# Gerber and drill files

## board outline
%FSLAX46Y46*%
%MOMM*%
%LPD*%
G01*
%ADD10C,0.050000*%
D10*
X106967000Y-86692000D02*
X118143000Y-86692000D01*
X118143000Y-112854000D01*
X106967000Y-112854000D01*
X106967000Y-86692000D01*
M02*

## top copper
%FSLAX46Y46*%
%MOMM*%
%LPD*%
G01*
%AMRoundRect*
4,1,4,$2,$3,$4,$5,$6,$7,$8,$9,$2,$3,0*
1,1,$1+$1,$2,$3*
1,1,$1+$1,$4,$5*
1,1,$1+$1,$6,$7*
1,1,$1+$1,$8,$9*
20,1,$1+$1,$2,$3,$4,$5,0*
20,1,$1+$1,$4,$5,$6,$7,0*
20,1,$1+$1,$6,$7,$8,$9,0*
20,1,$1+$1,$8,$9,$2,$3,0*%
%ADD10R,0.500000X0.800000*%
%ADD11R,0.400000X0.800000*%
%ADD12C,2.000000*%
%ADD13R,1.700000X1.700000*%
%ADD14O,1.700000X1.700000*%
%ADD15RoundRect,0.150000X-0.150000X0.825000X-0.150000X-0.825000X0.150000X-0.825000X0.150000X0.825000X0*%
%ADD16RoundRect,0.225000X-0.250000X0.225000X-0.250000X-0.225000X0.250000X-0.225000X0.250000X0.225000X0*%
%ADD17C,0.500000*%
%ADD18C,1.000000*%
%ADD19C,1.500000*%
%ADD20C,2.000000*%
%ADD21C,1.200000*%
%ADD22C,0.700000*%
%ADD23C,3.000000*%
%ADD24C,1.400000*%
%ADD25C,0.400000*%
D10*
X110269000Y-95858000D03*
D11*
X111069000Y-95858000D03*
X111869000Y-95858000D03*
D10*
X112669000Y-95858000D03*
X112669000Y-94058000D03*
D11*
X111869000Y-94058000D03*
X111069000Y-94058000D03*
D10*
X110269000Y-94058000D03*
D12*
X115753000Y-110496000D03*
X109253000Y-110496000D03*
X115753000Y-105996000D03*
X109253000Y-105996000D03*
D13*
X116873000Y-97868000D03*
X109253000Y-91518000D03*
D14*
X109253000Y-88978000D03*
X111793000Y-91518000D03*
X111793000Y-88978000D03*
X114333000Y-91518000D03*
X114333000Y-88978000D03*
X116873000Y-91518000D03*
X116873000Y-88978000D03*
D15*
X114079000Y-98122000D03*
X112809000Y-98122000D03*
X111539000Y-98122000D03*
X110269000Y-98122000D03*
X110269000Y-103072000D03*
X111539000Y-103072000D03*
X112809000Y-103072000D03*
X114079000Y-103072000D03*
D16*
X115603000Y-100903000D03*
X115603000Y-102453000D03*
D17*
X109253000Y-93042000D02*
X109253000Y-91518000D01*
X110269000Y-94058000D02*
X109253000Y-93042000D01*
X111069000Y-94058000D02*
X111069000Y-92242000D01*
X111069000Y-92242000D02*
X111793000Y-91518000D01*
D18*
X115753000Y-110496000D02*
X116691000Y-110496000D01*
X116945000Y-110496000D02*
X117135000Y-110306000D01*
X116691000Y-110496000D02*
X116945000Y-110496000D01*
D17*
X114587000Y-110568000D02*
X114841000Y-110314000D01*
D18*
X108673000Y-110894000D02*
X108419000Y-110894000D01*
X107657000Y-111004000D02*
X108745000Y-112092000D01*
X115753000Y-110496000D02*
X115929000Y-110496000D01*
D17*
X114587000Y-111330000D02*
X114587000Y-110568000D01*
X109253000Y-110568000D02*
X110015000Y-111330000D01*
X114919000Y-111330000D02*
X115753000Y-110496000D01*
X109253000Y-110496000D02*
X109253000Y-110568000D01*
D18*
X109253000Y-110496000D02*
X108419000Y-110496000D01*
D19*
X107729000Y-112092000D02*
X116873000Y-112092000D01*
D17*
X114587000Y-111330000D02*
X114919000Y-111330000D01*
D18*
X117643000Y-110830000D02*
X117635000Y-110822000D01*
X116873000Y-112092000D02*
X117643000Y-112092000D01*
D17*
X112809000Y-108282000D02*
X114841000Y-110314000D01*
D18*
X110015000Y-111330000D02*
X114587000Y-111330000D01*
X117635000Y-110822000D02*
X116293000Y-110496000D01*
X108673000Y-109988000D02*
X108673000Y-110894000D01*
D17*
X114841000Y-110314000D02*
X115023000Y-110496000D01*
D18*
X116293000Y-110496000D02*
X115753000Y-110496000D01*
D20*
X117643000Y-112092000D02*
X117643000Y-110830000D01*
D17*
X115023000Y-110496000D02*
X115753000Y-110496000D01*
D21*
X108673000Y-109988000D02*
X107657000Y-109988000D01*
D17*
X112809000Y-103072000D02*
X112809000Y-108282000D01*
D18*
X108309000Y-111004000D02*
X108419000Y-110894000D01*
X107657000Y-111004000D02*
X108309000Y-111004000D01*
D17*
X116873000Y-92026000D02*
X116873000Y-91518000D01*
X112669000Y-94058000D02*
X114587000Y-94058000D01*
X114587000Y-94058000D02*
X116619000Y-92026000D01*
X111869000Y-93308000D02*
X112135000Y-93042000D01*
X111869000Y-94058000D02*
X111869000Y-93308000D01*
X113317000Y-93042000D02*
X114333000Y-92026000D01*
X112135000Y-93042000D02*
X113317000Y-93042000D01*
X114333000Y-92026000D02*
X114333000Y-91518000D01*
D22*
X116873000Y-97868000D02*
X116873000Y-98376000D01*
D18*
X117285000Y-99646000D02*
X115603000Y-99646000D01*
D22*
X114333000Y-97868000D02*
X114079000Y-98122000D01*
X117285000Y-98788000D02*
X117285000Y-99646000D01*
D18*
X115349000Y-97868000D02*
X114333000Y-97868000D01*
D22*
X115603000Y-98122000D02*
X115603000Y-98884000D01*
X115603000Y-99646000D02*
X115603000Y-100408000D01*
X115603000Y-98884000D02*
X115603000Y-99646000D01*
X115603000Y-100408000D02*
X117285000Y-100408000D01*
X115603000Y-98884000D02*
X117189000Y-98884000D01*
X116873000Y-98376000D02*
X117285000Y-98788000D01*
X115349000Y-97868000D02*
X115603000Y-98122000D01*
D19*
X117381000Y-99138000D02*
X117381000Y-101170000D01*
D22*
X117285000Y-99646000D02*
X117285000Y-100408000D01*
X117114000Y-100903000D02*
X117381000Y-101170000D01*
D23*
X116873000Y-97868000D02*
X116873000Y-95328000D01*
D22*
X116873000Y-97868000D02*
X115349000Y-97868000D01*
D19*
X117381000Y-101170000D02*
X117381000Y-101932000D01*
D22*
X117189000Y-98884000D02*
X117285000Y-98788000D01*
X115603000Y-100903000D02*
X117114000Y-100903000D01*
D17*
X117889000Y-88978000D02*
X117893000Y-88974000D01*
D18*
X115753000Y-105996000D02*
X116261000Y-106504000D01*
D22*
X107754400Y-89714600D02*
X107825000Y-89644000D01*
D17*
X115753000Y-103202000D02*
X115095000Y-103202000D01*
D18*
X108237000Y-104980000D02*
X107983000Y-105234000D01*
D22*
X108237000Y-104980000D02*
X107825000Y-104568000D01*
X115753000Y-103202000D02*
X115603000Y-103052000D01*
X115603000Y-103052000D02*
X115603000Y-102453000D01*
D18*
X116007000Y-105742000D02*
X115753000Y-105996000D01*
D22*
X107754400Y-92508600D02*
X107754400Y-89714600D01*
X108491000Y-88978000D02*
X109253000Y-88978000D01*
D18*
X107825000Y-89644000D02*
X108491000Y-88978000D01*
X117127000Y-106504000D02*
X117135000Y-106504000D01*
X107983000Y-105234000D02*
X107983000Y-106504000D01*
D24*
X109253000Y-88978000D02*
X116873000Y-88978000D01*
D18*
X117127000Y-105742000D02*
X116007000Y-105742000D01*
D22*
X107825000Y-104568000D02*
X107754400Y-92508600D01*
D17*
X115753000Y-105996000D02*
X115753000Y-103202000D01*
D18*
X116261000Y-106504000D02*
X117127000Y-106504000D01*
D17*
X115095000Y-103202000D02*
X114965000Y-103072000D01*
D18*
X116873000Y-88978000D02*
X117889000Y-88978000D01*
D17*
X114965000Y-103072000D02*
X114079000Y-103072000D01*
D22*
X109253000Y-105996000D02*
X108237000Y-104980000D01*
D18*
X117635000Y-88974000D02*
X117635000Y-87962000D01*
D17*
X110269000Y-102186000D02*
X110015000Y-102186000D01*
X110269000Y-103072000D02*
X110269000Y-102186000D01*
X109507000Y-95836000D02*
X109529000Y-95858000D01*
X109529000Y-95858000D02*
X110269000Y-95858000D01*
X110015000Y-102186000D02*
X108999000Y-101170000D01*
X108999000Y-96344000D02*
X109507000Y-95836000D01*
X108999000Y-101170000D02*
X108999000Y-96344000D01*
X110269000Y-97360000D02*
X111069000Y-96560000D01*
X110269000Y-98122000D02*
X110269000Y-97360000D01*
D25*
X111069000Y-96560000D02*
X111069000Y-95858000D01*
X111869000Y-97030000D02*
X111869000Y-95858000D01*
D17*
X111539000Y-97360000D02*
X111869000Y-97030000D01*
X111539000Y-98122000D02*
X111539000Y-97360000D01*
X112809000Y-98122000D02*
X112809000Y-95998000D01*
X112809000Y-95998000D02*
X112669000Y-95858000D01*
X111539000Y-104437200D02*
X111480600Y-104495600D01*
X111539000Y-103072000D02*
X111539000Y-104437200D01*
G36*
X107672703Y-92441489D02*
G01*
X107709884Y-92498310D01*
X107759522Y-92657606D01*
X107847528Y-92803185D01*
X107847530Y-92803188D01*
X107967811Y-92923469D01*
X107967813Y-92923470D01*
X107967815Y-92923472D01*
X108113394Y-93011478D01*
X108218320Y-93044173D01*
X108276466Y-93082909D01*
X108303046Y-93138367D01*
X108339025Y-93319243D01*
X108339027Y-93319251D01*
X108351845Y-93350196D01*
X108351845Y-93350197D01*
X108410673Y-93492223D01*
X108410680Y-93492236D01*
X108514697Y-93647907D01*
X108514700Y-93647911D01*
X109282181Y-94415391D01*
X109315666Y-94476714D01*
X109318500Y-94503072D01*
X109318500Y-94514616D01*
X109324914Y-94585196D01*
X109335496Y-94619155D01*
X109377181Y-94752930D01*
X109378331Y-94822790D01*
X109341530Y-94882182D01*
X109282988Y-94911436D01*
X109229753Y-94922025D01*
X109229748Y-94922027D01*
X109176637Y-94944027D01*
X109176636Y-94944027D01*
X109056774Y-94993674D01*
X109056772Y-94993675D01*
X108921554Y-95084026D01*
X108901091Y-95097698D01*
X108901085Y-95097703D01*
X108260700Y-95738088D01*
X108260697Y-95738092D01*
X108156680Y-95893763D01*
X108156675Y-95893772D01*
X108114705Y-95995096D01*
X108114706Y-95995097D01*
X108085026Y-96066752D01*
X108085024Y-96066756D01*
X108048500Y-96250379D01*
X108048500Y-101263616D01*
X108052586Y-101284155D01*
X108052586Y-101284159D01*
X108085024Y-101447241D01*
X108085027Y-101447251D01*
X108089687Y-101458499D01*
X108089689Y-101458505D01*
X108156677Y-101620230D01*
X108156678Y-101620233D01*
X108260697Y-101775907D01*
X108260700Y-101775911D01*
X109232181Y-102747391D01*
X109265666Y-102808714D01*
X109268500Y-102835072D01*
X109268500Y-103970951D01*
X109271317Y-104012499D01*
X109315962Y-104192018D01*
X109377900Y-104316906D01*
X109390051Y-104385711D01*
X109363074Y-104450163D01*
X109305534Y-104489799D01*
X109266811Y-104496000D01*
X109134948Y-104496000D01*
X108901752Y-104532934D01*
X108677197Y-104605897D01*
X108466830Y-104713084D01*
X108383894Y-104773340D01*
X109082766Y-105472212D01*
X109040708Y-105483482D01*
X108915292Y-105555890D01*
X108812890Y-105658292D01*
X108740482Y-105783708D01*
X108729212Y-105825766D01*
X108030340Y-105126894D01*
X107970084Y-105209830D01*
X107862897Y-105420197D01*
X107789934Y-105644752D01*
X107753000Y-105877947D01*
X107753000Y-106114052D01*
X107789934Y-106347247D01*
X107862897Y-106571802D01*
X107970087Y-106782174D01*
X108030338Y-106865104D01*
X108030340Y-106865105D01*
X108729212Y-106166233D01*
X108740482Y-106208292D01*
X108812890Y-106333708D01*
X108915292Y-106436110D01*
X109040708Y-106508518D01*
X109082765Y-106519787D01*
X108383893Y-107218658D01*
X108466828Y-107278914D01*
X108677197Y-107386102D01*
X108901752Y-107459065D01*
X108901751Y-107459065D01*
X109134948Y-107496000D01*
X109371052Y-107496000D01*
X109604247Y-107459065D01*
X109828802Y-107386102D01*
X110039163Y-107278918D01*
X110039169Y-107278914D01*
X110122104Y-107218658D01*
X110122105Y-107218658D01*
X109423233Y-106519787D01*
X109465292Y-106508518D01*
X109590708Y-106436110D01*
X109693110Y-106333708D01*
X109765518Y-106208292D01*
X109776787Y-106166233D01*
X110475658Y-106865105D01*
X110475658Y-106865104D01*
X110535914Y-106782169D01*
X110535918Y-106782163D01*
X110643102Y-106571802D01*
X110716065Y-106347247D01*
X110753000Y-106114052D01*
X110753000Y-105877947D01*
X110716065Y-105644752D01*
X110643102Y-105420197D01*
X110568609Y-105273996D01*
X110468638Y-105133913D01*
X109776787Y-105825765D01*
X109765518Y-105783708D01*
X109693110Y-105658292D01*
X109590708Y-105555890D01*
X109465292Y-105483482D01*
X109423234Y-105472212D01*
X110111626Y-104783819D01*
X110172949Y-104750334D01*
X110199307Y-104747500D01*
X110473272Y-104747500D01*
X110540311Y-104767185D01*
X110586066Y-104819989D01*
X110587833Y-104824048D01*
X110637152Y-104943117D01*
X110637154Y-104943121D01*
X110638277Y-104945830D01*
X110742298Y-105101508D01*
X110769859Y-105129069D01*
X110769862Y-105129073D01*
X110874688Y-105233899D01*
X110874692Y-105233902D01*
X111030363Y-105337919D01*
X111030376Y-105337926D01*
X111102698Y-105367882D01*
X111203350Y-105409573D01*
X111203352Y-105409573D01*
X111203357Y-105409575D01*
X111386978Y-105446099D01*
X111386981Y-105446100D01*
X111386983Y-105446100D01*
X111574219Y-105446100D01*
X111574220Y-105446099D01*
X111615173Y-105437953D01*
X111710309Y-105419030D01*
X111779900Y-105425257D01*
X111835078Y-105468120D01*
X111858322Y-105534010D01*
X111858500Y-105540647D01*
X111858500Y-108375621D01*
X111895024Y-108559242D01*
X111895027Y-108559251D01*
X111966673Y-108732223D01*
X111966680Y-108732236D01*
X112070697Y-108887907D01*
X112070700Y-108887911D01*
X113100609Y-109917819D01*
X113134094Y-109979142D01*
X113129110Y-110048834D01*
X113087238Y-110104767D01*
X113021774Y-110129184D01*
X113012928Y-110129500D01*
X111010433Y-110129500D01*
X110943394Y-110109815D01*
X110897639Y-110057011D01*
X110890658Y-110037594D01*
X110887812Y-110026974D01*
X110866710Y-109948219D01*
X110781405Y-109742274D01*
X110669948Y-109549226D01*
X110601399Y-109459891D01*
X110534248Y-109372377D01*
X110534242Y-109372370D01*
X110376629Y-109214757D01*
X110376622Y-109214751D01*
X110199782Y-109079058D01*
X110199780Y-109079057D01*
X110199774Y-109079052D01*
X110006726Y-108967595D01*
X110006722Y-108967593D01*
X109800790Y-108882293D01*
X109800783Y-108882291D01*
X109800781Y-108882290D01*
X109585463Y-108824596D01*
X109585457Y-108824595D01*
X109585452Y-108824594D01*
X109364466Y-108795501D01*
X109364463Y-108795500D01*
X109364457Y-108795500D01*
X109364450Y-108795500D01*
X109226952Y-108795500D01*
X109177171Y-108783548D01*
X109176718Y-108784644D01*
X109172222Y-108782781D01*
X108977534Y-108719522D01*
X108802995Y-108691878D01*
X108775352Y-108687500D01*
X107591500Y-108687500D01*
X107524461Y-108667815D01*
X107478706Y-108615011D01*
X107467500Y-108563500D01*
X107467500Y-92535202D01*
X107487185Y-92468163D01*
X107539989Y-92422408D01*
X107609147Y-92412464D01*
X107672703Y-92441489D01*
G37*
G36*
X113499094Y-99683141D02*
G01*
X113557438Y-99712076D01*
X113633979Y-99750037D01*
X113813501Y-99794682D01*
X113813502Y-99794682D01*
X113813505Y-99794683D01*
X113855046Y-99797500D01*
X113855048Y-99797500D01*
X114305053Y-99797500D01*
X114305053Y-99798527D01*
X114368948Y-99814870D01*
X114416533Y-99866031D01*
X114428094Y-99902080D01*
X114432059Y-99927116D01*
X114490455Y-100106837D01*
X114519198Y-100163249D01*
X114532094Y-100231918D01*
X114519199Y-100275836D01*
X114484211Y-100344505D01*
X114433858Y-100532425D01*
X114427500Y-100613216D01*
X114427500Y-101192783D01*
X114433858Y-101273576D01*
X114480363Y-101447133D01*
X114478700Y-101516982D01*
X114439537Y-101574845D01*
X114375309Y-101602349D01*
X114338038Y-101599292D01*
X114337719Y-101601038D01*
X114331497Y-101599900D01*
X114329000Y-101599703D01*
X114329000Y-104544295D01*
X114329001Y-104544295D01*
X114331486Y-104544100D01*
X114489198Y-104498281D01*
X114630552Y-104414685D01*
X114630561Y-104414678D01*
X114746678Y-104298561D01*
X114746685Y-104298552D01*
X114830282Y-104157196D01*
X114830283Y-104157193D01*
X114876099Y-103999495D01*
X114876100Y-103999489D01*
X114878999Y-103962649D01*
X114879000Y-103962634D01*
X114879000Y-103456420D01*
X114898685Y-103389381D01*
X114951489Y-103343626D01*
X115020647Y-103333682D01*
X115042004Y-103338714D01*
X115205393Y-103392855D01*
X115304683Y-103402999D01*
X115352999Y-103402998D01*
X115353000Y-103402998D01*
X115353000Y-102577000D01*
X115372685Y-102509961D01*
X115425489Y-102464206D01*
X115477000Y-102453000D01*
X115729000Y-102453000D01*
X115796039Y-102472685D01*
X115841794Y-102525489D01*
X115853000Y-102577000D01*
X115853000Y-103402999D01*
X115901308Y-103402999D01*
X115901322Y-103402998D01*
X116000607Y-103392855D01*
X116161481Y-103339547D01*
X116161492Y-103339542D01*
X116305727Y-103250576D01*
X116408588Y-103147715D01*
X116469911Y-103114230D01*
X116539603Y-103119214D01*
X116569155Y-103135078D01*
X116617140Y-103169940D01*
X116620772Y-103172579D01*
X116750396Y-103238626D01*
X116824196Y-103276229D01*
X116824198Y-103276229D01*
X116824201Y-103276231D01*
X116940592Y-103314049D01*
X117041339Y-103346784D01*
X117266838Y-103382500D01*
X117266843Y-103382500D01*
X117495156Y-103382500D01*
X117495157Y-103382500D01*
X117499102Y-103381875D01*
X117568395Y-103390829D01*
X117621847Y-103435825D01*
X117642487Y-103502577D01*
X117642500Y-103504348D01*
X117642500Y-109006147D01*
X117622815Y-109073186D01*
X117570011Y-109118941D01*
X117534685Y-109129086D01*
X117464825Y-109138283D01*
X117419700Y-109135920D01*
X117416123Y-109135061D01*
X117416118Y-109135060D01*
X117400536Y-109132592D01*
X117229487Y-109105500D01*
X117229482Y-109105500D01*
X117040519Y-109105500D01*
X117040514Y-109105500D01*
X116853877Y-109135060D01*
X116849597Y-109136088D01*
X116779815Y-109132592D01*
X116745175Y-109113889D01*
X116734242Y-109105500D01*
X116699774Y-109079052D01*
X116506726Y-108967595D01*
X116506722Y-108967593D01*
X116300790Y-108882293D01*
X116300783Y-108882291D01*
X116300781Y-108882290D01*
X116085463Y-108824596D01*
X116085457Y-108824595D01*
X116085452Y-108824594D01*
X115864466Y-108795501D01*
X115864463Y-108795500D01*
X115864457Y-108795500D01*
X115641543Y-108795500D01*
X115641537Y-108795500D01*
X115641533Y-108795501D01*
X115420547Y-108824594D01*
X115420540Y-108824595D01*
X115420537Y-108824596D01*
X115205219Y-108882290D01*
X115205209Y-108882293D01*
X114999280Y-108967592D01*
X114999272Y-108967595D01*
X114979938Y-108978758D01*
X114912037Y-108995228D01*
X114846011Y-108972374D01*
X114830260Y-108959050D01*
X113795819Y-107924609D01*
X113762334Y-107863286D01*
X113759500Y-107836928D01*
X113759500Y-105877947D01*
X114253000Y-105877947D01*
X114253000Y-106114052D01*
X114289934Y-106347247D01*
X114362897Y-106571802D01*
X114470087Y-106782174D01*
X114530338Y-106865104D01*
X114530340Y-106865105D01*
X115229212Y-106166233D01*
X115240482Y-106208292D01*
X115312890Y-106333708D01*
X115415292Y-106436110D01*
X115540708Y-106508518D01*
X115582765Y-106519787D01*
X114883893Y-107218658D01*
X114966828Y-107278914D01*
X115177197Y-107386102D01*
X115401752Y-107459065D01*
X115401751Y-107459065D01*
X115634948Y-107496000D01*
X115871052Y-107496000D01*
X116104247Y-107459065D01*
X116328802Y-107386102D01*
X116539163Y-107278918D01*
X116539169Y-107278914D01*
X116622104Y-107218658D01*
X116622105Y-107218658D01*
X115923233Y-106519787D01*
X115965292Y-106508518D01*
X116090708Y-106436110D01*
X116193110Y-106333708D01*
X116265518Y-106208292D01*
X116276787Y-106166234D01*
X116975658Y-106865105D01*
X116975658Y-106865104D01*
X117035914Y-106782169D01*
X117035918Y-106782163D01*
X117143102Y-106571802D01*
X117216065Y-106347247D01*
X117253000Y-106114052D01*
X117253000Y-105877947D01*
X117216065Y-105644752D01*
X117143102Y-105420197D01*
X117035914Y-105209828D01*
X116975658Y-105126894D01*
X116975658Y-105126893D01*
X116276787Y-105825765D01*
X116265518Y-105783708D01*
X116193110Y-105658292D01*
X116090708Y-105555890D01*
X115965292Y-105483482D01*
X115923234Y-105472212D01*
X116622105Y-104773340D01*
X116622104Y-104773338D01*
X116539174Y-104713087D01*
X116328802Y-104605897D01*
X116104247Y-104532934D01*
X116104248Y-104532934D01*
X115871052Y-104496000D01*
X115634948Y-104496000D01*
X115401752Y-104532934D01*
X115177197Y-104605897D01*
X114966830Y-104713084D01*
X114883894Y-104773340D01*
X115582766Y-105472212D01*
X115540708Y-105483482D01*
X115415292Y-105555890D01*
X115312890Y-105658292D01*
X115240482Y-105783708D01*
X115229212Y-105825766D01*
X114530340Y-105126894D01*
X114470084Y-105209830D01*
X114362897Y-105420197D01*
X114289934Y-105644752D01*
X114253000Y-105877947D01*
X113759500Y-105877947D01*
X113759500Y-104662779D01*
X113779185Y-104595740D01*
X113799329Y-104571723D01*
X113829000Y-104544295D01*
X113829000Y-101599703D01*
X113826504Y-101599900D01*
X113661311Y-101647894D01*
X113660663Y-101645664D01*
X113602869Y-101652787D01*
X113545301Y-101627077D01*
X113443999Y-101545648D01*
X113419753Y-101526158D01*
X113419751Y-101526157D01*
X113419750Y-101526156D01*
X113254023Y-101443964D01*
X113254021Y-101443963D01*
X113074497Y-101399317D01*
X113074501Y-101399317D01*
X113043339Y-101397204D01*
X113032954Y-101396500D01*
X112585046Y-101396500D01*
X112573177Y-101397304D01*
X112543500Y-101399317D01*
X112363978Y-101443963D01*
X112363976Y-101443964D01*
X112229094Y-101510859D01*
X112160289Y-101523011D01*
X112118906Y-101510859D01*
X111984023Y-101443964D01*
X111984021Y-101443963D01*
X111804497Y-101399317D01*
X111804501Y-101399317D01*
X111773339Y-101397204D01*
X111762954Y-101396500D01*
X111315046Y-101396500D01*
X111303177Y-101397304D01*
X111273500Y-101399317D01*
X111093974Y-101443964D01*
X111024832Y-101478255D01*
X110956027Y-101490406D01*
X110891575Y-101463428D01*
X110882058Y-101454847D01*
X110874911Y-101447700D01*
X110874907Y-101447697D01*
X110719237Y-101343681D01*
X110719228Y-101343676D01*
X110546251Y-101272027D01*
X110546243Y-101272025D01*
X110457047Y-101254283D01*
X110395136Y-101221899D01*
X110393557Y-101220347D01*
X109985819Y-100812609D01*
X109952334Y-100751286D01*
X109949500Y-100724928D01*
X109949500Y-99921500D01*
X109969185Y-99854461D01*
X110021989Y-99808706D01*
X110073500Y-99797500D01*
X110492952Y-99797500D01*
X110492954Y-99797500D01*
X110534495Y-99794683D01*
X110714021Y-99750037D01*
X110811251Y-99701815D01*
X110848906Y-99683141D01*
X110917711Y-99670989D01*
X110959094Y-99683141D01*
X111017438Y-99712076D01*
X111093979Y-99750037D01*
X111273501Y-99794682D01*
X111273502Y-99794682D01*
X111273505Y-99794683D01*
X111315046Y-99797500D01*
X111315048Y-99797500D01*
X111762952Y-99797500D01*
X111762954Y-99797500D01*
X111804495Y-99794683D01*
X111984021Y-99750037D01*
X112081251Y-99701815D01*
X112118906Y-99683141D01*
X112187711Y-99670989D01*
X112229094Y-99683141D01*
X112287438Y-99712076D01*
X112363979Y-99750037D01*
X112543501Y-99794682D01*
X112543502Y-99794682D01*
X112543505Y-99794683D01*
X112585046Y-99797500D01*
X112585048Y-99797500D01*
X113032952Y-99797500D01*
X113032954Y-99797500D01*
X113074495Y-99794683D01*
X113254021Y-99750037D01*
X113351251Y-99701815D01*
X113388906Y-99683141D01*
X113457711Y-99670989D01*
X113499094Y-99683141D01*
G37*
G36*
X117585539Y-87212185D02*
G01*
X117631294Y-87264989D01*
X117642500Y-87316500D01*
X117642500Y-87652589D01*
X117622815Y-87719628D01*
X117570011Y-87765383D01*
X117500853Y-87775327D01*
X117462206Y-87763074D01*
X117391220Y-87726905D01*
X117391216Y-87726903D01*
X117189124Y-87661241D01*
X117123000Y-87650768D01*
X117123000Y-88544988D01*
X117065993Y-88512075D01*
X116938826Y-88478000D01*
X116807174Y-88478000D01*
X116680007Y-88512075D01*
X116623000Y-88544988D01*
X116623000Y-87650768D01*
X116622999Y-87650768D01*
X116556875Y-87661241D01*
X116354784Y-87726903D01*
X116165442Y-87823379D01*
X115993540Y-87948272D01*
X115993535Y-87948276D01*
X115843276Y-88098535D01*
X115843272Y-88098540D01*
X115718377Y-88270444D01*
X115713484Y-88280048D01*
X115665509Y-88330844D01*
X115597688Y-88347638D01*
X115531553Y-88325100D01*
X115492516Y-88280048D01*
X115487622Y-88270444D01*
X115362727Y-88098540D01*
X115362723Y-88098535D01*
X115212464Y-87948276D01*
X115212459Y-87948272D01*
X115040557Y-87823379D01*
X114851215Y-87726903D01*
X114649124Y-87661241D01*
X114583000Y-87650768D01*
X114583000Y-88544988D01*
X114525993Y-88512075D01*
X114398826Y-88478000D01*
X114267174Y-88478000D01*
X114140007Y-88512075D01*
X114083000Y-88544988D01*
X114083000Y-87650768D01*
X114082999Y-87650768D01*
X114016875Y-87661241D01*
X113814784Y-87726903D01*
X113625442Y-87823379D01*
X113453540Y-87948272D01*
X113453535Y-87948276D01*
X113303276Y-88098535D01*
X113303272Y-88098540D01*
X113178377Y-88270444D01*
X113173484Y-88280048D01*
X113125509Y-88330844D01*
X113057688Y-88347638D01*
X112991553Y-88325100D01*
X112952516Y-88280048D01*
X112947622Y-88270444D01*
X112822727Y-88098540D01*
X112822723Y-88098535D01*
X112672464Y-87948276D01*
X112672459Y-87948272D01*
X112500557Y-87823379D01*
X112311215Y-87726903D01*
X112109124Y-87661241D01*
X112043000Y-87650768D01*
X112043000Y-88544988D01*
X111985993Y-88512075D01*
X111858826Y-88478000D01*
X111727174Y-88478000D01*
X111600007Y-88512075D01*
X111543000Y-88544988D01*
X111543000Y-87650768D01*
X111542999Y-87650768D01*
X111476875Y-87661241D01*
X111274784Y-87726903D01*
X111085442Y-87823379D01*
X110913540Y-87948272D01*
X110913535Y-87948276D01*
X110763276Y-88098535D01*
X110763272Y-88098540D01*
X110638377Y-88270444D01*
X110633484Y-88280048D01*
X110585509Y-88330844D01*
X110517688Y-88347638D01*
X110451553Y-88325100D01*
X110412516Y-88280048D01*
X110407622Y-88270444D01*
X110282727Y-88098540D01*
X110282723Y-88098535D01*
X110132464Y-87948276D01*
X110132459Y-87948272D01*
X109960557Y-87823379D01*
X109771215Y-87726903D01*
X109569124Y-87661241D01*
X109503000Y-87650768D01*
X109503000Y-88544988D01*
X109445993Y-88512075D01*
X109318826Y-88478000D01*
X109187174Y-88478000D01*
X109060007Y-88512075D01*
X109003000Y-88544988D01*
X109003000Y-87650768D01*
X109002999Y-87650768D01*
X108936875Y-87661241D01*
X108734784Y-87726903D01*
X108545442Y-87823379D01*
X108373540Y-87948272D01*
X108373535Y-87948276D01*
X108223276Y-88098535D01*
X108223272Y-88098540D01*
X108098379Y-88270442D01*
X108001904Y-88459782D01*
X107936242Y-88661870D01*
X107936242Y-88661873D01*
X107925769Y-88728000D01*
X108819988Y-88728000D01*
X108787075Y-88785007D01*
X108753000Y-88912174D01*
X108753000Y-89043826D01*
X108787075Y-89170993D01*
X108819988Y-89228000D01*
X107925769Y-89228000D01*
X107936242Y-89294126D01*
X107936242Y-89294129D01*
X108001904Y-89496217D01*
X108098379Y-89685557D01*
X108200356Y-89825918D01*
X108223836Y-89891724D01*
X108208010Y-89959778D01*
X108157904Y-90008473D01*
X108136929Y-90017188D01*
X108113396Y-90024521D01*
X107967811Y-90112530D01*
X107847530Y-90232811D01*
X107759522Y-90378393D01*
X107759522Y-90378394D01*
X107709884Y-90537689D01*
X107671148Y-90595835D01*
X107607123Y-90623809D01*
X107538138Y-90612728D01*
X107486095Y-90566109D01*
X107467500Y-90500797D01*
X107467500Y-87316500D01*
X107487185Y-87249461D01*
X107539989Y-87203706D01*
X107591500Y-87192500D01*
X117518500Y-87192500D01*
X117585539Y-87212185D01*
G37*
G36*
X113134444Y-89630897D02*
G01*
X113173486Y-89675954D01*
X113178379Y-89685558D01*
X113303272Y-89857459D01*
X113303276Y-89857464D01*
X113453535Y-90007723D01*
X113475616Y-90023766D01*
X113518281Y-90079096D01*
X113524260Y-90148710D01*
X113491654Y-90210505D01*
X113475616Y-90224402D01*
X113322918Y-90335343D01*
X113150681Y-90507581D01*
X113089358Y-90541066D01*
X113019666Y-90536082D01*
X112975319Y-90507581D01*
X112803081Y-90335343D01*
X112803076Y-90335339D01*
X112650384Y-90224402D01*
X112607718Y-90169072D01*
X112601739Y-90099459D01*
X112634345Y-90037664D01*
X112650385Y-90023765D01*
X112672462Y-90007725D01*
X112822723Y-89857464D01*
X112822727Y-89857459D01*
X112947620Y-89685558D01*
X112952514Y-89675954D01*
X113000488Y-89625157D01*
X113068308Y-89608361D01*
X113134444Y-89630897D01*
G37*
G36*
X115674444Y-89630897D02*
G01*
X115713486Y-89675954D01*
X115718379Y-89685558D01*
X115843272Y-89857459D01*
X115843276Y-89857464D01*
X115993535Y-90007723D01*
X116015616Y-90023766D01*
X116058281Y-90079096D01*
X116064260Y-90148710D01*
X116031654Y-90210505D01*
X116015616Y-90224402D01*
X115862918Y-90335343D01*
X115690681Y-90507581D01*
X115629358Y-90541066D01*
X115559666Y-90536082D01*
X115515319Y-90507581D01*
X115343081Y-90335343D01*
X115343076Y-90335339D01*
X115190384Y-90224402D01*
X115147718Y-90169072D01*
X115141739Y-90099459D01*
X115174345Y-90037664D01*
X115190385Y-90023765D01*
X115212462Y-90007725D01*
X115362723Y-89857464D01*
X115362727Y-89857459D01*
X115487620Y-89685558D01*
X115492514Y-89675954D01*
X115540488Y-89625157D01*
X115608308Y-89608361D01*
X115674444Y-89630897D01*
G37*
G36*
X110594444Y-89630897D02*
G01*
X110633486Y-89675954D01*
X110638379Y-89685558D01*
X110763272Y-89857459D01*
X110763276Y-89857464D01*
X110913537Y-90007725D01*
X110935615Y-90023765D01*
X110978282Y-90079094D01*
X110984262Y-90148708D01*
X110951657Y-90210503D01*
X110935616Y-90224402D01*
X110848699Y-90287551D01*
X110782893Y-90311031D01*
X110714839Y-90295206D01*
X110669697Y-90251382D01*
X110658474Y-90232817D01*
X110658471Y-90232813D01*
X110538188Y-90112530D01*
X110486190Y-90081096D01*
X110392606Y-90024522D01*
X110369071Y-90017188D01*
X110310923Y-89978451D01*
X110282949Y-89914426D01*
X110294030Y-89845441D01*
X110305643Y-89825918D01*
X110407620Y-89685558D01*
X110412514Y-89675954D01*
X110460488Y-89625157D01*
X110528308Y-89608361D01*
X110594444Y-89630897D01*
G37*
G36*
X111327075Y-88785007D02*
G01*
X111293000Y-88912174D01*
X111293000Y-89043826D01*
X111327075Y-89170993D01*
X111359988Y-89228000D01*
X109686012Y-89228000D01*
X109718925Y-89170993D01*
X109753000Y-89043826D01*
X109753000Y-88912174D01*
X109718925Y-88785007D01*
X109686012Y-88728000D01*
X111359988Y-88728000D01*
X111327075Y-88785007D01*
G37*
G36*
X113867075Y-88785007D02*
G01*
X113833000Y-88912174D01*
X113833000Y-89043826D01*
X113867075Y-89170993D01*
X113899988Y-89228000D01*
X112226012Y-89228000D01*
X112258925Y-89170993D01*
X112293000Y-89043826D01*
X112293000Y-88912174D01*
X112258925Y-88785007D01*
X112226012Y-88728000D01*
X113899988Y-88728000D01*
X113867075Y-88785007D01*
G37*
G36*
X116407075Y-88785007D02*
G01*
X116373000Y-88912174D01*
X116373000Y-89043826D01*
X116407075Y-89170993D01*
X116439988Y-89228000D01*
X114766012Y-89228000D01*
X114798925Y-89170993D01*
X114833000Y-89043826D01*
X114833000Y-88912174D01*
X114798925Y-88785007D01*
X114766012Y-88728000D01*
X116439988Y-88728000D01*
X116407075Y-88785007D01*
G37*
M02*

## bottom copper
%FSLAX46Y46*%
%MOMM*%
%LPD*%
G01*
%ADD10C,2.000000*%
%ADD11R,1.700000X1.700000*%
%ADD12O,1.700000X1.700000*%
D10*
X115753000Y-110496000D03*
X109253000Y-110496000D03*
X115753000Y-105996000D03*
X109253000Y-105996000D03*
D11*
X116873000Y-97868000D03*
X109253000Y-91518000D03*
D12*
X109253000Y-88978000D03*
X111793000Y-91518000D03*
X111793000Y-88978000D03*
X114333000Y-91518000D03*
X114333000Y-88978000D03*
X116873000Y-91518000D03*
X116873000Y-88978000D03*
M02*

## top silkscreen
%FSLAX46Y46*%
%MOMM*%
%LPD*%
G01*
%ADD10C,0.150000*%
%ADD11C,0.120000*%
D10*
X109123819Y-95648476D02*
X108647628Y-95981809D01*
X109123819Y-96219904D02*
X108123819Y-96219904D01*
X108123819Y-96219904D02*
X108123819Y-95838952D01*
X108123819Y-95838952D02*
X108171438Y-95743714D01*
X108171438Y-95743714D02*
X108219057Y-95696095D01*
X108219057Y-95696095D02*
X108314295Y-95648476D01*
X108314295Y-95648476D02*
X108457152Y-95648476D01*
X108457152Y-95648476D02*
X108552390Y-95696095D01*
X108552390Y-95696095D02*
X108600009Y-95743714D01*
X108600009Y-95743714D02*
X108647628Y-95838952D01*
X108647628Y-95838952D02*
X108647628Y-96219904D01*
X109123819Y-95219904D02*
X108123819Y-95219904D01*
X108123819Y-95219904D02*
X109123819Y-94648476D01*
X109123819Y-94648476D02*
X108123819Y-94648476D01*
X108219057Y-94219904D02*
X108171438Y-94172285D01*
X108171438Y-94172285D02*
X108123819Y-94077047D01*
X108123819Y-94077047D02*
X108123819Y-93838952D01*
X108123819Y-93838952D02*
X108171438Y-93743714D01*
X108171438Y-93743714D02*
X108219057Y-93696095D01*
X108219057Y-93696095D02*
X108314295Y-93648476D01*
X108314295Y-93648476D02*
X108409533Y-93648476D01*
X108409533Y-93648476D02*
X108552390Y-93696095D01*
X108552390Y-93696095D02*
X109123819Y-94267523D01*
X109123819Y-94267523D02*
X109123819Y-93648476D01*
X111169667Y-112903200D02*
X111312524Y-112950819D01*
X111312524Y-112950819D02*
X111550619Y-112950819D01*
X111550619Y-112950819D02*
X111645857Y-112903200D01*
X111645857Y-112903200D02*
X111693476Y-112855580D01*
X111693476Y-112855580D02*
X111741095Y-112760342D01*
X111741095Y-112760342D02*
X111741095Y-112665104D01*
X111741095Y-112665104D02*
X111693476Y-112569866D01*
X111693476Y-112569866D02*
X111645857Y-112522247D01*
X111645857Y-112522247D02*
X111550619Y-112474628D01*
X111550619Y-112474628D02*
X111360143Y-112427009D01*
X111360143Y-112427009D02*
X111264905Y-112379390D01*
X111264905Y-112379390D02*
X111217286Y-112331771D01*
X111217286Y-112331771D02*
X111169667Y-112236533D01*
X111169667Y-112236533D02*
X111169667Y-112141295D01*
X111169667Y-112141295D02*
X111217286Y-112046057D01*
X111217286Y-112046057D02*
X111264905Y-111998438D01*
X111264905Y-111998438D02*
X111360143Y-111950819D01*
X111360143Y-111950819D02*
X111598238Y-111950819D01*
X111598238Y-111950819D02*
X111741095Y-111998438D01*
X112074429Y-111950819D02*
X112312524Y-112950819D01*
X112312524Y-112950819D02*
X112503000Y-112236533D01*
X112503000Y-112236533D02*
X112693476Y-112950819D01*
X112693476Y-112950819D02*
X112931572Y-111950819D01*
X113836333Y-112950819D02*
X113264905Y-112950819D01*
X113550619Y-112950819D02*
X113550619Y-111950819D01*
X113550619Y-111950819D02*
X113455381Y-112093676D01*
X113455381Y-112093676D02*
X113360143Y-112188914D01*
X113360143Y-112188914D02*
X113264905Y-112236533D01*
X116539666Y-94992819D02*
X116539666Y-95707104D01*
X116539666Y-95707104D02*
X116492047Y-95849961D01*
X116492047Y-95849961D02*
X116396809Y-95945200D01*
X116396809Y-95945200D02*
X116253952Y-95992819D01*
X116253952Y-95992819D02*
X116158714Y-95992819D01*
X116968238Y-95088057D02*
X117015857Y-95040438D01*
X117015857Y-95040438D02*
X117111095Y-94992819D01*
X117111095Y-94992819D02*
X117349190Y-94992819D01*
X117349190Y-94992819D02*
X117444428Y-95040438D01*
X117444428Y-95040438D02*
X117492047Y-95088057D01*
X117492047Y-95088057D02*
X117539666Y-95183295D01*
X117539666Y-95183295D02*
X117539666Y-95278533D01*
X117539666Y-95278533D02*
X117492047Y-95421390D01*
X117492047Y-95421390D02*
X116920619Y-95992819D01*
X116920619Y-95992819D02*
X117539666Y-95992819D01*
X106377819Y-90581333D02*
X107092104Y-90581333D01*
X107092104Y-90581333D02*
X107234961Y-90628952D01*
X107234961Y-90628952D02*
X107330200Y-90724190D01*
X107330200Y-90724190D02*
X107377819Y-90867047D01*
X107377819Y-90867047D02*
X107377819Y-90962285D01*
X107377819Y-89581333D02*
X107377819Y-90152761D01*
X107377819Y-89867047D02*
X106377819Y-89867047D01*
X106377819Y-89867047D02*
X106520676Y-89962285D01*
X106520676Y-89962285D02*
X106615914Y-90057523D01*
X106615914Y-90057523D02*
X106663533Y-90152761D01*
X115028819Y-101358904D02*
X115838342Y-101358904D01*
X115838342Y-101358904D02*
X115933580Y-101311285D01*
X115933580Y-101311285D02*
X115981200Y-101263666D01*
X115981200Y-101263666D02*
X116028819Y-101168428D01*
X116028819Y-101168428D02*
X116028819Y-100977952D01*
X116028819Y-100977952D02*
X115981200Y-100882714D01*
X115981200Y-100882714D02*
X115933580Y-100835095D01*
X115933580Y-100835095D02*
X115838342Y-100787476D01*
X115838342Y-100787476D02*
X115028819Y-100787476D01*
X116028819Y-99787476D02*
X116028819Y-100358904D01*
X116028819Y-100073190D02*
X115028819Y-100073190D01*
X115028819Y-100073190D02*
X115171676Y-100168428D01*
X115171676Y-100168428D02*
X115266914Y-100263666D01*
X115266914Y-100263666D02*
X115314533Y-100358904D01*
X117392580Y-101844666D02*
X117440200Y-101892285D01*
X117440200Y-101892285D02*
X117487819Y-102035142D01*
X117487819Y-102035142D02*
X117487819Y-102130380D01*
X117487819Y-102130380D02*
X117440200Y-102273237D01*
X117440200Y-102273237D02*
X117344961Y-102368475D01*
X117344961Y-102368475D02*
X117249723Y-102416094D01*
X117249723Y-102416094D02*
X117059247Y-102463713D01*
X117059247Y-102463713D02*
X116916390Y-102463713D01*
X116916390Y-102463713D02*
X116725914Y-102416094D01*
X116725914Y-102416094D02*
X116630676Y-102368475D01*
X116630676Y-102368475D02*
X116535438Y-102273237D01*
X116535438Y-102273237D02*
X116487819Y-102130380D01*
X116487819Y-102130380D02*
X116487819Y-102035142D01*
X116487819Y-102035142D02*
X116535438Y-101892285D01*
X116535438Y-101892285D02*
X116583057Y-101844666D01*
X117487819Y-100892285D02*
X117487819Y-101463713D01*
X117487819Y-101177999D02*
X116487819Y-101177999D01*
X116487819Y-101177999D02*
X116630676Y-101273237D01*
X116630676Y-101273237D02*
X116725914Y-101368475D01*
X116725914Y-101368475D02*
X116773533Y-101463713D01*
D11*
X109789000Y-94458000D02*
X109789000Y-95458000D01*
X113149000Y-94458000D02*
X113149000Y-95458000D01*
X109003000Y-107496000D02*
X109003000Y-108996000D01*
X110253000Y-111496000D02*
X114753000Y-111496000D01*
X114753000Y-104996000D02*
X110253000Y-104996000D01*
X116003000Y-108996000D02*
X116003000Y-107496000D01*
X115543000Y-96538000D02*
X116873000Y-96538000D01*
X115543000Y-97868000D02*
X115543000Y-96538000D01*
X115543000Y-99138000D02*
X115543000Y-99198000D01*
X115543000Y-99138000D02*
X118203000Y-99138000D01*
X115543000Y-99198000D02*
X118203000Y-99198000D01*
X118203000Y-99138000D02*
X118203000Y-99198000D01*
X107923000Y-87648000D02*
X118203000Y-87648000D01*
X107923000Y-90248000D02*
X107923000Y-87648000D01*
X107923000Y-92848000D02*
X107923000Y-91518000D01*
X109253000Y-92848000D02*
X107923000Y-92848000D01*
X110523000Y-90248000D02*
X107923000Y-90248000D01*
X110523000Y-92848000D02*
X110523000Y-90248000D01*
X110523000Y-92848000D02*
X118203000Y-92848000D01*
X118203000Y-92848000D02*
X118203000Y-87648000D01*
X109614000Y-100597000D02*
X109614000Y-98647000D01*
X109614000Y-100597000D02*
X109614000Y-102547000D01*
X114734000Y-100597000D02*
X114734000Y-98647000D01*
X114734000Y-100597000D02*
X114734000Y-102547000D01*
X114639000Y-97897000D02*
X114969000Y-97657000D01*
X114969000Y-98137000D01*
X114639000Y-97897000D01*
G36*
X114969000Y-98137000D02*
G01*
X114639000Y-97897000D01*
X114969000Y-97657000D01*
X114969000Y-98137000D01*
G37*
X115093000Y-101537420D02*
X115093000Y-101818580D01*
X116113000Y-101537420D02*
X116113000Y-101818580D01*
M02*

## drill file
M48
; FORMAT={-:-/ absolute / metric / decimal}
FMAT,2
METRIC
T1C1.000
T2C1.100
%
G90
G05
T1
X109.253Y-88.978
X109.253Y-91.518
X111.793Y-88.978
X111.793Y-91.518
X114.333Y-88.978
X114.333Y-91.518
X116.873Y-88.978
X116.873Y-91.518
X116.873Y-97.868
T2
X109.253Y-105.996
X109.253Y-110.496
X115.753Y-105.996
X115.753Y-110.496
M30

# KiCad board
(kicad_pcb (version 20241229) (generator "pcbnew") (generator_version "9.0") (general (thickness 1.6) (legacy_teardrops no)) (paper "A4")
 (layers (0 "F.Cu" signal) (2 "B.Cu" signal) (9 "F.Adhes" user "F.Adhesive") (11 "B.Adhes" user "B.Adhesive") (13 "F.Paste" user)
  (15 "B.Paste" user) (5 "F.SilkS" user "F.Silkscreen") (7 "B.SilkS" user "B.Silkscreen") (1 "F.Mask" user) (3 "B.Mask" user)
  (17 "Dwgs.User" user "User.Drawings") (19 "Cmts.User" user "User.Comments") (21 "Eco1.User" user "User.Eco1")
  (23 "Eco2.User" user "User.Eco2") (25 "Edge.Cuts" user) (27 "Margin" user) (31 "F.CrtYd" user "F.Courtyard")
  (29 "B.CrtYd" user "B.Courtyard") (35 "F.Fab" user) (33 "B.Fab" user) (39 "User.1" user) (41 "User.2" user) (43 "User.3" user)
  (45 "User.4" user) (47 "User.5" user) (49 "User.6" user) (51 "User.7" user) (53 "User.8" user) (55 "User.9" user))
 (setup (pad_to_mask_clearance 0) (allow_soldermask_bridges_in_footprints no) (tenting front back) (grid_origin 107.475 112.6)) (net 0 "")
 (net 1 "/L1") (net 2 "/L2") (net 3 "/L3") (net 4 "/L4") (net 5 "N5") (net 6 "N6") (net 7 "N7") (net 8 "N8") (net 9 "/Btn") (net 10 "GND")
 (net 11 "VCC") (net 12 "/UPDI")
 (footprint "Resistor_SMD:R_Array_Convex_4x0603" (layer "F.Cu") (at 111.469 94.958 90)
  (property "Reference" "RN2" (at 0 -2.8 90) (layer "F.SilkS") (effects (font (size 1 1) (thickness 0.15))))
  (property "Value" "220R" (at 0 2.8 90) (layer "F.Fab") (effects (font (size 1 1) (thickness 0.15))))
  (fp_line (start 0.5 -1.68) (end -0.5 -1.68) (stroke (width 0.12) (type solid)) (layer "F.SilkS"))
  (fp_line (start 0.5 1.68) (end -0.5 1.68) (stroke (width 0.12) (type solid)) (layer "F.SilkS"))
  (pad "1" smd rect (at -0.9 -1.2 90) (size 0.8 0.5) (layers "F.Cu" "F.Mask" "F.Paste") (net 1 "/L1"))
  (pad "2" smd rect (at -0.9 -0.4 90) (size 0.8 0.4) (layers "F.Cu" "F.Mask" "F.Paste") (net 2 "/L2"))
  (pad "3" smd rect (at -0.9 0.4 90) (size 0.8 0.4) (layers "F.Cu" "F.Mask" "F.Paste") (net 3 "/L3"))
  (pad "4" smd rect (at -0.9 1.2 90) (size 0.8 0.5) (layers "F.Cu" "F.Mask" "F.Paste") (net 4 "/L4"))
  (pad "5" smd rect (at 0.9 1.2 90) (size 0.8 0.5) (layers "F.Cu" "F.Mask" "F.Paste") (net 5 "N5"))
  (pad "6" smd rect (at 0.9 0.4 90) (size 0.8 0.4) (layers "F.Cu" "F.Mask" "F.Paste") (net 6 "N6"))
  (pad "7" smd rect (at 0.9 -0.4 90) (size 0.8 0.4) (layers "F.Cu" "F.Mask" "F.Paste") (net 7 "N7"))
  (pad "8" smd rect (at 0.9 -1.2 90) (size 0.8 0.5) (layers "F.Cu" "F.Mask" "F.Paste") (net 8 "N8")))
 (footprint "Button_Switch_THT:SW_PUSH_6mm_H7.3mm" (layer "F.Cu") (at 115.753 110.496 180)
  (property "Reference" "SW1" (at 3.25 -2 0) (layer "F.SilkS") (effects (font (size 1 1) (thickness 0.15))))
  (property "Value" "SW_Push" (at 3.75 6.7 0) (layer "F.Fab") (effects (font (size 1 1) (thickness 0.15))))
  (fp_line (start 6.75 3) (end 6.75 1.5) (stroke (width 0.12) (type solid)) (layer "F.SilkS"))
  (fp_line (start 5.5 -1) (end 1 -1) (stroke (width 0.12) (type solid)) (layer "F.SilkS"))
  (fp_line (start 1 5.5) (end 5.5 5.5) (stroke (width 0.12) (type solid)) (layer "F.SilkS"))
  (fp_line (start -0.25 1.5) (end -0.25 3) (stroke (width 0.12) (type solid)) (layer "F.SilkS"))
  (pad "1" thru_hole circle (at 0 0 270) (size 2 2) (drill 1.1) (layers "*.Cu" "*.Mask") (remove_unused_layers no) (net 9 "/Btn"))
  (pad "1" thru_hole circle (at 6.5 0 270) (size 2 2) (drill 1.1) (layers "*.Cu" "*.Mask") (remove_unused_layers no) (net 9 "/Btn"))
  (pad "2" thru_hole circle (at 0 4.5 270) (size 2 2) (drill 1.1) (layers "*.Cu" "*.Mask") (remove_unused_layers no) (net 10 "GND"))
  (pad "2" thru_hole circle (at 6.5 4.5 270) (size 2 2) (drill 1.1) (layers "*.Cu" "*.Mask") (remove_unused_layers no) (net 10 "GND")))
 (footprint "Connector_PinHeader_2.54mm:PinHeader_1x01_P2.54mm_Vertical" (layer "F.Cu") (at 116.873 97.868)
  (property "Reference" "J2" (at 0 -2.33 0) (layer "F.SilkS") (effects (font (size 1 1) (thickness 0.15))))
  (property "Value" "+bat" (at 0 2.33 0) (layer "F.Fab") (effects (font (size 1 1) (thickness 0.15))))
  (fp_line (start -1.33 -1.33) (end 0 -1.33) (stroke (width 0.12) (type solid)) (layer "F.SilkS"))
  (fp_line (start -1.33 0) (end -1.33 -1.33) (stroke (width 0.12) (type solid)) (layer "F.SilkS"))
  (fp_line (start -1.33 1.27) (end -1.33 1.33) (stroke (width 0.12) (type solid)) (layer "F.SilkS"))
  (fp_line (start -1.33 1.27) (end 1.33 1.27) (stroke (width 0.12) (type solid)) (layer "F.SilkS"))
  (fp_line (start -1.33 1.33) (end 1.33 1.33) (stroke (width 0.12) (type solid)) (layer "F.SilkS"))
  (fp_line (start 1.33 1.27) (end 1.33 1.33) (stroke (width 0.12) (type solid)) (layer "F.SilkS"))
  (pad "1" thru_hole rect (at 0 0) (size 1.7 1.7) (drill 1) (layers "*.Cu" "*.Mask") (remove_unused_layers no) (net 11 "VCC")))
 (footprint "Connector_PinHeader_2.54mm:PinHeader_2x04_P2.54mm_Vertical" (layer "F.Cu") (at 109.253 91.518 90)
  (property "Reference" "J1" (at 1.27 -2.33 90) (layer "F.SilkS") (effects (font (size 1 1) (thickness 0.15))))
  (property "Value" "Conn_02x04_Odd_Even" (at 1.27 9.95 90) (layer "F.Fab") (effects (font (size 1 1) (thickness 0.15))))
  (fp_line (start 3.87 -1.33) (end 3.87 8.95) (stroke (width 0.12) (type solid)) (layer "F.SilkS"))
  (fp_line (start 1.27 -1.33) (end 3.87 -1.33) (stroke (width 0.12) (type solid)) (layer "F.SilkS"))
  (fp_line (start -1.33 -1.33) (end 0 -1.33) (stroke (width 0.12) (type solid)) (layer "F.SilkS"))
  (fp_line (start -1.33 0) (end -1.33 -1.33) (stroke (width 0.12) (type solid)) (layer "F.SilkS"))
  (fp_line (start 1.27 1.27) (end 1.27 -1.33) (stroke (width 0.12) (type solid)) (layer "F.SilkS"))
  (fp_line (start -1.33 1.27) (end 1.27 1.27) (stroke (width 0.12) (type solid)) (layer "F.SilkS"))
  (fp_line (start -1.33 1.27) (end -1.33 8.95) (stroke (width 0.12) (type solid)) (layer "F.SilkS"))
  (fp_line (start -1.33 8.95) (end 3.87 8.95) (stroke (width 0.12) (type solid)) (layer "F.SilkS"))
  (pad "1" thru_hole rect (at 0 0 90) (size 1.7 1.7) (drill 1) (layers "*.Cu" "*.Mask") (remove_unused_layers no) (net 8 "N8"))
  (pad "2" thru_hole oval (at 2.54 0 90) (size 1.7 1.7) (drill 1) (layers "*.Cu" "*.Mask") (remove_unused_layers no) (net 10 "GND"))
  (pad "3" thru_hole oval (at 0 2.54 90) (size 1.7 1.7) (drill 1) (layers "*.Cu" "*.Mask") (remove_unused_layers no) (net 7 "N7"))
  (pad "4" thru_hole oval (at 2.54 2.54 90) (size 1.7 1.7) (drill 1) (layers "*.Cu" "*.Mask") (remove_unused_layers no) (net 10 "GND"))
  (pad "5" thru_hole oval (at 0 5.08 90) (size 1.7 1.7) (drill 1) (layers "*.Cu" "*.Mask") (remove_unused_layers no) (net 6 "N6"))
  (pad "6" thru_hole oval (at 2.54 5.08 90) (size 1.7 1.7) (drill 1) (layers "*.Cu" "*.Mask") (remove_unused_layers no) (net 10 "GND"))
  (pad "7" thru_hole oval (at 0 7.62 90) (size 1.7 1.7) (drill 1) (layers "*.Cu" "*.Mask") (remove_unused_layers no) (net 5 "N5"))
  (pad "8" thru_hole oval (at 2.54 7.62 90) (size 1.7 1.7) (drill 1) (layers "*.Cu" "*.Mask") (remove_unused_layers no) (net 10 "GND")))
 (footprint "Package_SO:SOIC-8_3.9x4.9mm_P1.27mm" (layer "F.Cu") (at 112.174 100.597 -90)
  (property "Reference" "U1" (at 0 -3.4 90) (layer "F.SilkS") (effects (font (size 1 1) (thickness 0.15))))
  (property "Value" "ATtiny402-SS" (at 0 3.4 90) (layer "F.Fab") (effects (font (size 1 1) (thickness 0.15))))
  (fp_line (start 0 2.56) (end -1.95 2.56) (stroke (width 0.12) (type solid)) (layer "F.SilkS"))
  (fp_line (start 0 2.56) (end 1.95 2.56) (stroke (width 0.12) (type solid)) (layer "F.SilkS"))
  (fp_line (start 0 -2.56) (end -1.95 -2.56) (stroke (width 0.12) (type solid)) (layer "F.SilkS"))
  (fp_line (start 0 -2.56) (end 1.95 -2.56) (stroke (width 0.12) (type solid)) (layer "F.SilkS"))
  (fp_poly
   (pts (xy -2.7 -2.465) (xy -2.94 -2.795) (xy -2.46 -2.795) (xy -2.7 -2.465)) (stroke (width 0.12) (type solid)) (fill yes)
   (layer "F.SilkS"))
  (pad "1" smd roundrect (at -2.475 -1.905 270) (size 1.95 0.6) (layers "F.Cu" "F.Mask" "F.Paste") (roundrect_rratio 0.25) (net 11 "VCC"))
  (pad "2" smd roundrect (at -2.475 -0.635 270) (size 1.95 0.6) (layers "F.Cu" "F.Mask" "F.Paste") (roundrect_rratio 0.25) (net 4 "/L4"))
  (pad "3" smd roundrect (at -2.475 0.635 270) (size 1.95 0.6) (layers "F.Cu" "F.Mask" "F.Paste") (roundrect_rratio 0.25) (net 3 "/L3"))
  (pad "4" smd roundrect (at -2.475 1.905 270) (size 1.95 0.6) (layers "F.Cu" "F.Mask" "F.Paste") (roundrect_rratio 0.25) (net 2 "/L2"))
  (pad "5" smd roundrect (at 2.475 1.905 270) (size 1.95 0.6) (layers "F.Cu" "F.Mask" "F.Paste") (roundrect_rratio 0.25) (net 1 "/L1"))
  (pad "6" smd roundrect (at 2.475 0.635 270) (size 1.95 0.6) (layers "F.Cu" "F.Mask" "F.Paste") (roundrect_rratio 0.25) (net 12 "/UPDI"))
  (pad "7" smd roundrect (at 2.475 -0.635 270) (size 1.95 0.6) (layers "F.Cu" "F.Mask" "F.Paste") (roundrect_rratio 0.25) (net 9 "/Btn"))
  (pad "8" smd roundrect (at 2.475 -1.905 270) (size 1.95 0.6) (layers "F.Cu" "F.Mask" "F.Paste") (roundrect_rratio 0.25) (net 10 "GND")))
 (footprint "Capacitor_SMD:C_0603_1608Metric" (layer "F.Cu") (at 115.603 101.678 -90)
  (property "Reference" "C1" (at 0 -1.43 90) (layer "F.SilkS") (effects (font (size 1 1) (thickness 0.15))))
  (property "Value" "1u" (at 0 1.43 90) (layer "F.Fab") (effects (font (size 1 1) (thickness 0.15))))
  (fp_line (start -0.14058 0.51) (end 0.14058 0.51) (stroke (width 0.12) (type solid)) (layer "F.SilkS"))
  (fp_line (start -0.14058 -0.51) (end 0.14058 -0.51) (stroke (width 0.12) (type solid)) (layer "F.SilkS"))
  (pad "1" smd roundrect (at -0.775 0 270) (size 0.9 0.95) (layers "F.Cu" "F.Mask" "F.Paste") (roundrect_rratio 0.25) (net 11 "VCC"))
  (pad "2" smd roundrect (at 0.775 0 270) (size 0.9 0.95) (layers "F.Cu" "F.Mask" "F.Paste") (roundrect_rratio 0.25) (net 10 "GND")))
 (gr_rect (start 106.967 86.692) (end 118.143 112.854) (stroke (width 0.05) (type default)) (fill no) (layer "Edge.Cuts"))
 (segment (start 109.253 93.042) (end 109.253 91.518) (width 0.5) (layer "F.Cu") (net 8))
 (segment (start 110.269 94.058) (end 109.253 93.042) (width 0.5) (layer "F.Cu") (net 8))
 (segment (start 111.069 94.058) (end 111.069 92.242) (width 0.5) (layer "F.Cu") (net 7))
 (segment (start 111.069 92.242) (end 111.793 91.518) (width 0.5) (layer "F.Cu") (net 7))
 (segment (start 115.753 110.496) (end 116.691 110.496) (width 1) (layer "F.Cu") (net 9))
 (segment (start 116.945 110.496) (end 117.135 110.306) (width 1) (layer "F.Cu") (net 9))
 (segment (start 116.691 110.496) (end 116.945 110.496) (width 1) (layer "F.Cu") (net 9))
 (segment (start 114.587 110.568) (end 114.841 110.314) (width 0.5) (layer "F.Cu") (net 9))
 (segment (start 108.673 110.894) (end 108.419 110.894) (width 1) (layer "F.Cu") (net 9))
 (segment (start 107.657 111.004) (end 108.745 112.092) (width 1) (layer "F.Cu") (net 9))
 (segment (start 115.753 110.496) (end 115.929 110.496) (width 1) (layer "F.Cu") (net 9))
 (segment (start 114.587 111.33) (end 114.587 110.568) (width 0.5) (layer "F.Cu") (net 9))
 (segment (start 109.253 110.568) (end 110.015 111.33) (width 0.5) (layer "F.Cu") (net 9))
 (segment (start 114.919 111.33) (end 115.753 110.496) (width 0.5) (layer "F.Cu") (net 9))
 (segment (start 109.253 110.496) (end 109.253 110.568) (width 0.5) (layer "F.Cu") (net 9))
 (segment (start 109.253 110.496) (end 108.419 110.496) (width 1) (layer "F.Cu") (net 9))
 (segment (start 107.729 112.092) (end 116.873 112.092) (width 1.5) (layer "F.Cu") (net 9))
 (segment (start 114.587 111.33) (end 114.919 111.33) (width 0.5) (layer "F.Cu") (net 9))
 (segment (start 117.643 110.83) (end 117.635 110.822) (width 1) (layer "F.Cu") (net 9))
 (segment (start 116.873 112.092) (end 117.643 112.092) (width 1) (layer "F.Cu") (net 9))
 (segment (start 112.809 108.282) (end 114.841 110.314) (width 0.5) (layer "F.Cu") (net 9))
 (segment (start 110.015 111.33) (end 114.587 111.33) (width 1) (layer "F.Cu") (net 9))
 (segment (start 117.635 110.822) (end 116.293 110.496) (width 1) (layer "F.Cu") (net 9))
 (segment (start 108.673 109.988) (end 108.673 110.894) (width 1) (layer "F.Cu") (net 9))
 (segment (start 114.841 110.314) (end 115.023 110.496) (width 0.5) (layer "F.Cu") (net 9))
 (segment (start 116.293 110.496) (end 115.753 110.496) (width 1) (layer "F.Cu") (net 9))
 (segment (start 117.643 112.092) (end 117.643 110.83) (width 2) (layer "F.Cu") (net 9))
 (segment (start 115.023 110.496) (end 115.753 110.496) (width 0.5) (layer "F.Cu") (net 9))
 (segment (start 108.673 109.988) (end 107.657 109.988) (width 1.2) (layer "F.Cu") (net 9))
 (segment (start 112.809 103.072) (end 112.809 108.282) (width 0.5) (layer "F.Cu") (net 9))
 (segment (start 108.309 111.004) (end 108.419 110.894) (width 1) (layer "F.Cu") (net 9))
 (segment (start 107.657 111.004) (end 108.309 111.004) (width 1) (layer "F.Cu") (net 9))
 (segment (start 116.873 92.026) (end 116.873 91.518) (width 0.5) (layer "F.Cu") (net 5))
 (segment (start 112.669 94.058) (end 114.587 94.058) (width 0.5) (layer "F.Cu") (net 5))
 (segment (start 114.587 94.058) (end 116.619 92.026) (width 0.5) (layer "F.Cu") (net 5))
 (segment (start 111.869 93.308) (end 112.135 93.042) (width 0.5) (layer "F.Cu") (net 6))
 (segment (start 111.869 94.058) (end 111.869 93.308) (width 0.5) (layer "F.Cu") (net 6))
 (segment (start 113.317 93.042) (end 114.333 92.026) (width 0.5) (layer "F.Cu") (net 6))
 (segment (start 112.135 93.042) (end 113.317 93.042) (width 0.5) (layer "F.Cu") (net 6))
 (segment (start 114.333 92.026) (end 114.333 91.518) (width 0.5) (layer "F.Cu") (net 6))
 (segment (start 116.873 97.868) (end 116.873 98.376) (width 0.7) (layer "F.Cu") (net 11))
 (segment (start 117.285 99.646) (end 115.603 99.646) (width 1) (layer "F.Cu") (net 11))
 (segment (start 114.333 97.868) (end 114.079 98.122) (width 0.7) (layer "F.Cu") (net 11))
 (segment (start 117.285 98.788) (end 117.285 99.646) (width 0.7) (layer "F.Cu") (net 11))
 (segment (start 115.349 97.868) (end 114.333 97.868) (width 1) (layer "F.Cu") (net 11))
 (segment (start 115.603 98.122) (end 115.603 98.884) (width 0.7) (layer "F.Cu") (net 11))
 (segment (start 115.603 99.646) (end 115.603 100.408) (width 0.7) (layer "F.Cu") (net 11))
 (segment (start 115.603 98.884) (end 115.603 99.646) (width 0.7) (layer "F.Cu") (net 11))
 (segment (start 115.603 100.408) (end 117.285 100.408) (width 0.7) (layer "F.Cu") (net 11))
 (segment (start 115.603 98.884) (end 117.189 98.884) (width 0.7) (layer "F.Cu") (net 11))
 (segment (start 116.873 98.376) (end 117.285 98.788) (width 0.7) (layer "F.Cu") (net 11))
 (segment (start 115.349 97.868) (end 115.603 98.122) (width 0.7) (layer "F.Cu") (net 11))
 (segment (start 117.381 99.138) (end 117.381 101.17) (width 1.5) (layer "F.Cu") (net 11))
 (segment (start 117.285 99.646) (end 117.285 100.408) (width 0.7) (layer "F.Cu") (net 11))
 (segment (start 117.114 100.903) (end 117.381 101.17) (width 0.7) (layer "F.Cu") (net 11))
 (segment (start 116.873 97.868) (end 116.873 95.328) (width 3) (layer "F.Cu") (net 11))
 (segment (start 116.873 97.868) (end 115.349 97.868) (width 0.7) (layer "F.Cu") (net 11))
 (segment (start 117.381 101.17) (end 117.381 101.932) (width 1.5) (layer "F.Cu") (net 11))
 (segment (start 117.189 98.884) (end 117.285 98.788) (width 0.7) (layer "F.Cu") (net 11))
 (segment (start 115.603 100.903) (end 117.114 100.903) (width 0.7) (layer "F.Cu") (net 11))
 (segment (start 117.889 88.978) (end 117.893 88.974) (width 0.5) (layer "F.Cu") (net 10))
 (segment (start 115.753 105.996) (end 116.261 106.504) (width 1) (layer "F.Cu") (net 10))
 (segment (start 107.7544 89.7146) (end 107.825 89.644) (width 0.7) (layer "F.Cu") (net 10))
 (segment (start 115.753 103.202) (end 115.095 103.202) (width 0.5) (layer "F.Cu") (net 10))
 (segment (start 108.237 104.98) (end 107.983 105.234) (width 1) (layer "F.Cu") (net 10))
 (segment (start 108.237 104.98) (end 107.825 104.568) (width 0.7) (layer "F.Cu") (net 10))
 (segment (start 115.753 103.202) (end 115.603 103.052) (width 0.7) (layer "F.Cu") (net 10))
 (segment (start 115.603 103.052) (end 115.603 102.453) (width 0.7) (layer "F.Cu") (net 10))
 (segment (start 116.007 105.742) (end 115.753 105.996) (width 1) (layer "F.Cu") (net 10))
 (segment (start 107.7544 92.5086) (end 107.7544 89.7146) (width 0.7) (layer "F.Cu") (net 10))
 (segment (start 108.491 88.978) (end 109.253 88.978) (width 0.7) (layer "F.Cu") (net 10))
 (segment (start 107.825 89.644) (end 108.491 88.978) (width 1) (layer "F.Cu") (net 10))
 (segment (start 117.127 106.504) (end 117.135 106.504) (width 1) (layer "F.Cu") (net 10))
 (segment (start 107.983 105.234) (end 107.983 106.504) (width 1) (layer "F.Cu") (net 10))
 (segment (start 109.253 88.978) (end 116.873 88.978) (width 1.4) (layer "F.Cu") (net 10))
 (segment (start 117.127 105.742) (end 116.007 105.742) (width 1) (layer "F.Cu") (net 10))
 (segment (start 107.825 104.568) (end 107.7544 92.5086) (width 0.7) (layer "F.Cu") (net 10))
 (segment (start 115.753 105.996) (end 115.753 103.202) (width 0.5) (layer "F.Cu") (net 10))
 (segment (start 116.261 106.504) (end 117.127 106.504) (width 1) (layer "F.Cu") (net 10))
 (segment (start 115.095 103.202) (end 114.965 103.072) (width 0.5) (layer "F.Cu") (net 10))
 (segment (start 116.873 88.978) (end 117.889 88.978) (width 1) (layer "F.Cu") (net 10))
 (segment (start 114.965 103.072) (end 114.079 103.072) (width 0.5) (layer "F.Cu") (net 10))
 (segment (start 109.253 105.996) (end 108.237 104.98) (width 0.7) (layer "F.Cu") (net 10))
 (segment (start 117.635 88.974) (end 117.635 87.962) (width 1) (layer "F.Cu") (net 10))
 (segment (start 110.269 102.186) (end 110.015 102.186) (width 0.5) (layer "F.Cu") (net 1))
 (segment (start 110.269 103.072) (end 110.269 102.186) (width 0.5) (layer "F.Cu") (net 1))
 (segment (start 109.507 95.836) (end 109.529 95.858) (width 0.5) (layer "F.Cu") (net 1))
 (segment (start 109.529 95.858) (end 110.269 95.858) (width 0.5) (layer "F.Cu") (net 1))
 (segment (start 110.015 102.186) (end 108.999 101.17) (width 0.5) (layer "F.Cu") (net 1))
 (segment (start 108.999 96.344) (end 109.507 95.836) (width 0.5) (layer "F.Cu") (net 1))
 (segment (start 108.999 101.17) (end 108.999 96.344) (width 0.5) (layer "F.Cu") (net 1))
 (segment (start 110.269 97.36) (end 111.069 96.56) (width 0.5) (layer "F.Cu") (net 2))
 (segment (start 110.269 98.122) (end 110.269 97.36) (width 0.5) (layer "F.Cu") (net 2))
 (segment (start 111.069 96.56) (end 111.069 95.858) (width 0.4) (layer "F.Cu") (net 2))
 (segment (start 111.869 97.03) (end 111.869 95.858) (width 0.4) (layer "F.Cu") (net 3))
 (segment (start 111.539 97.36) (end 111.869 97.03) (width 0.5) (layer "F.Cu") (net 3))
 (segment (start 111.539 98.122) (end 111.539 97.36) (width 0.5) (layer "F.Cu") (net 3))
 (segment (start 112.809 98.122) (end 112.809 95.998) (width 0.5) (layer "F.Cu") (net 4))
 (segment (start 112.809 95.998) (end 112.669 95.858) (width 0.5) (layer "F.Cu") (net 4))
 (segment (start 111.539 104.4372) (end 111.4806 104.4956) (width 0.5) (layer "F.Cu") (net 12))
 (segment (start 111.539 103.072) (end 111.539 104.4372) (width 0.5) (layer "F.Cu") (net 12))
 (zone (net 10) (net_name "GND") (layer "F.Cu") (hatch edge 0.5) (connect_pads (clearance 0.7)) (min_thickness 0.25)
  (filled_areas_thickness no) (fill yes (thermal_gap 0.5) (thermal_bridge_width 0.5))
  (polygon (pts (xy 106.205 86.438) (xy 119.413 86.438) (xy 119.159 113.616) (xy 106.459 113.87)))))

